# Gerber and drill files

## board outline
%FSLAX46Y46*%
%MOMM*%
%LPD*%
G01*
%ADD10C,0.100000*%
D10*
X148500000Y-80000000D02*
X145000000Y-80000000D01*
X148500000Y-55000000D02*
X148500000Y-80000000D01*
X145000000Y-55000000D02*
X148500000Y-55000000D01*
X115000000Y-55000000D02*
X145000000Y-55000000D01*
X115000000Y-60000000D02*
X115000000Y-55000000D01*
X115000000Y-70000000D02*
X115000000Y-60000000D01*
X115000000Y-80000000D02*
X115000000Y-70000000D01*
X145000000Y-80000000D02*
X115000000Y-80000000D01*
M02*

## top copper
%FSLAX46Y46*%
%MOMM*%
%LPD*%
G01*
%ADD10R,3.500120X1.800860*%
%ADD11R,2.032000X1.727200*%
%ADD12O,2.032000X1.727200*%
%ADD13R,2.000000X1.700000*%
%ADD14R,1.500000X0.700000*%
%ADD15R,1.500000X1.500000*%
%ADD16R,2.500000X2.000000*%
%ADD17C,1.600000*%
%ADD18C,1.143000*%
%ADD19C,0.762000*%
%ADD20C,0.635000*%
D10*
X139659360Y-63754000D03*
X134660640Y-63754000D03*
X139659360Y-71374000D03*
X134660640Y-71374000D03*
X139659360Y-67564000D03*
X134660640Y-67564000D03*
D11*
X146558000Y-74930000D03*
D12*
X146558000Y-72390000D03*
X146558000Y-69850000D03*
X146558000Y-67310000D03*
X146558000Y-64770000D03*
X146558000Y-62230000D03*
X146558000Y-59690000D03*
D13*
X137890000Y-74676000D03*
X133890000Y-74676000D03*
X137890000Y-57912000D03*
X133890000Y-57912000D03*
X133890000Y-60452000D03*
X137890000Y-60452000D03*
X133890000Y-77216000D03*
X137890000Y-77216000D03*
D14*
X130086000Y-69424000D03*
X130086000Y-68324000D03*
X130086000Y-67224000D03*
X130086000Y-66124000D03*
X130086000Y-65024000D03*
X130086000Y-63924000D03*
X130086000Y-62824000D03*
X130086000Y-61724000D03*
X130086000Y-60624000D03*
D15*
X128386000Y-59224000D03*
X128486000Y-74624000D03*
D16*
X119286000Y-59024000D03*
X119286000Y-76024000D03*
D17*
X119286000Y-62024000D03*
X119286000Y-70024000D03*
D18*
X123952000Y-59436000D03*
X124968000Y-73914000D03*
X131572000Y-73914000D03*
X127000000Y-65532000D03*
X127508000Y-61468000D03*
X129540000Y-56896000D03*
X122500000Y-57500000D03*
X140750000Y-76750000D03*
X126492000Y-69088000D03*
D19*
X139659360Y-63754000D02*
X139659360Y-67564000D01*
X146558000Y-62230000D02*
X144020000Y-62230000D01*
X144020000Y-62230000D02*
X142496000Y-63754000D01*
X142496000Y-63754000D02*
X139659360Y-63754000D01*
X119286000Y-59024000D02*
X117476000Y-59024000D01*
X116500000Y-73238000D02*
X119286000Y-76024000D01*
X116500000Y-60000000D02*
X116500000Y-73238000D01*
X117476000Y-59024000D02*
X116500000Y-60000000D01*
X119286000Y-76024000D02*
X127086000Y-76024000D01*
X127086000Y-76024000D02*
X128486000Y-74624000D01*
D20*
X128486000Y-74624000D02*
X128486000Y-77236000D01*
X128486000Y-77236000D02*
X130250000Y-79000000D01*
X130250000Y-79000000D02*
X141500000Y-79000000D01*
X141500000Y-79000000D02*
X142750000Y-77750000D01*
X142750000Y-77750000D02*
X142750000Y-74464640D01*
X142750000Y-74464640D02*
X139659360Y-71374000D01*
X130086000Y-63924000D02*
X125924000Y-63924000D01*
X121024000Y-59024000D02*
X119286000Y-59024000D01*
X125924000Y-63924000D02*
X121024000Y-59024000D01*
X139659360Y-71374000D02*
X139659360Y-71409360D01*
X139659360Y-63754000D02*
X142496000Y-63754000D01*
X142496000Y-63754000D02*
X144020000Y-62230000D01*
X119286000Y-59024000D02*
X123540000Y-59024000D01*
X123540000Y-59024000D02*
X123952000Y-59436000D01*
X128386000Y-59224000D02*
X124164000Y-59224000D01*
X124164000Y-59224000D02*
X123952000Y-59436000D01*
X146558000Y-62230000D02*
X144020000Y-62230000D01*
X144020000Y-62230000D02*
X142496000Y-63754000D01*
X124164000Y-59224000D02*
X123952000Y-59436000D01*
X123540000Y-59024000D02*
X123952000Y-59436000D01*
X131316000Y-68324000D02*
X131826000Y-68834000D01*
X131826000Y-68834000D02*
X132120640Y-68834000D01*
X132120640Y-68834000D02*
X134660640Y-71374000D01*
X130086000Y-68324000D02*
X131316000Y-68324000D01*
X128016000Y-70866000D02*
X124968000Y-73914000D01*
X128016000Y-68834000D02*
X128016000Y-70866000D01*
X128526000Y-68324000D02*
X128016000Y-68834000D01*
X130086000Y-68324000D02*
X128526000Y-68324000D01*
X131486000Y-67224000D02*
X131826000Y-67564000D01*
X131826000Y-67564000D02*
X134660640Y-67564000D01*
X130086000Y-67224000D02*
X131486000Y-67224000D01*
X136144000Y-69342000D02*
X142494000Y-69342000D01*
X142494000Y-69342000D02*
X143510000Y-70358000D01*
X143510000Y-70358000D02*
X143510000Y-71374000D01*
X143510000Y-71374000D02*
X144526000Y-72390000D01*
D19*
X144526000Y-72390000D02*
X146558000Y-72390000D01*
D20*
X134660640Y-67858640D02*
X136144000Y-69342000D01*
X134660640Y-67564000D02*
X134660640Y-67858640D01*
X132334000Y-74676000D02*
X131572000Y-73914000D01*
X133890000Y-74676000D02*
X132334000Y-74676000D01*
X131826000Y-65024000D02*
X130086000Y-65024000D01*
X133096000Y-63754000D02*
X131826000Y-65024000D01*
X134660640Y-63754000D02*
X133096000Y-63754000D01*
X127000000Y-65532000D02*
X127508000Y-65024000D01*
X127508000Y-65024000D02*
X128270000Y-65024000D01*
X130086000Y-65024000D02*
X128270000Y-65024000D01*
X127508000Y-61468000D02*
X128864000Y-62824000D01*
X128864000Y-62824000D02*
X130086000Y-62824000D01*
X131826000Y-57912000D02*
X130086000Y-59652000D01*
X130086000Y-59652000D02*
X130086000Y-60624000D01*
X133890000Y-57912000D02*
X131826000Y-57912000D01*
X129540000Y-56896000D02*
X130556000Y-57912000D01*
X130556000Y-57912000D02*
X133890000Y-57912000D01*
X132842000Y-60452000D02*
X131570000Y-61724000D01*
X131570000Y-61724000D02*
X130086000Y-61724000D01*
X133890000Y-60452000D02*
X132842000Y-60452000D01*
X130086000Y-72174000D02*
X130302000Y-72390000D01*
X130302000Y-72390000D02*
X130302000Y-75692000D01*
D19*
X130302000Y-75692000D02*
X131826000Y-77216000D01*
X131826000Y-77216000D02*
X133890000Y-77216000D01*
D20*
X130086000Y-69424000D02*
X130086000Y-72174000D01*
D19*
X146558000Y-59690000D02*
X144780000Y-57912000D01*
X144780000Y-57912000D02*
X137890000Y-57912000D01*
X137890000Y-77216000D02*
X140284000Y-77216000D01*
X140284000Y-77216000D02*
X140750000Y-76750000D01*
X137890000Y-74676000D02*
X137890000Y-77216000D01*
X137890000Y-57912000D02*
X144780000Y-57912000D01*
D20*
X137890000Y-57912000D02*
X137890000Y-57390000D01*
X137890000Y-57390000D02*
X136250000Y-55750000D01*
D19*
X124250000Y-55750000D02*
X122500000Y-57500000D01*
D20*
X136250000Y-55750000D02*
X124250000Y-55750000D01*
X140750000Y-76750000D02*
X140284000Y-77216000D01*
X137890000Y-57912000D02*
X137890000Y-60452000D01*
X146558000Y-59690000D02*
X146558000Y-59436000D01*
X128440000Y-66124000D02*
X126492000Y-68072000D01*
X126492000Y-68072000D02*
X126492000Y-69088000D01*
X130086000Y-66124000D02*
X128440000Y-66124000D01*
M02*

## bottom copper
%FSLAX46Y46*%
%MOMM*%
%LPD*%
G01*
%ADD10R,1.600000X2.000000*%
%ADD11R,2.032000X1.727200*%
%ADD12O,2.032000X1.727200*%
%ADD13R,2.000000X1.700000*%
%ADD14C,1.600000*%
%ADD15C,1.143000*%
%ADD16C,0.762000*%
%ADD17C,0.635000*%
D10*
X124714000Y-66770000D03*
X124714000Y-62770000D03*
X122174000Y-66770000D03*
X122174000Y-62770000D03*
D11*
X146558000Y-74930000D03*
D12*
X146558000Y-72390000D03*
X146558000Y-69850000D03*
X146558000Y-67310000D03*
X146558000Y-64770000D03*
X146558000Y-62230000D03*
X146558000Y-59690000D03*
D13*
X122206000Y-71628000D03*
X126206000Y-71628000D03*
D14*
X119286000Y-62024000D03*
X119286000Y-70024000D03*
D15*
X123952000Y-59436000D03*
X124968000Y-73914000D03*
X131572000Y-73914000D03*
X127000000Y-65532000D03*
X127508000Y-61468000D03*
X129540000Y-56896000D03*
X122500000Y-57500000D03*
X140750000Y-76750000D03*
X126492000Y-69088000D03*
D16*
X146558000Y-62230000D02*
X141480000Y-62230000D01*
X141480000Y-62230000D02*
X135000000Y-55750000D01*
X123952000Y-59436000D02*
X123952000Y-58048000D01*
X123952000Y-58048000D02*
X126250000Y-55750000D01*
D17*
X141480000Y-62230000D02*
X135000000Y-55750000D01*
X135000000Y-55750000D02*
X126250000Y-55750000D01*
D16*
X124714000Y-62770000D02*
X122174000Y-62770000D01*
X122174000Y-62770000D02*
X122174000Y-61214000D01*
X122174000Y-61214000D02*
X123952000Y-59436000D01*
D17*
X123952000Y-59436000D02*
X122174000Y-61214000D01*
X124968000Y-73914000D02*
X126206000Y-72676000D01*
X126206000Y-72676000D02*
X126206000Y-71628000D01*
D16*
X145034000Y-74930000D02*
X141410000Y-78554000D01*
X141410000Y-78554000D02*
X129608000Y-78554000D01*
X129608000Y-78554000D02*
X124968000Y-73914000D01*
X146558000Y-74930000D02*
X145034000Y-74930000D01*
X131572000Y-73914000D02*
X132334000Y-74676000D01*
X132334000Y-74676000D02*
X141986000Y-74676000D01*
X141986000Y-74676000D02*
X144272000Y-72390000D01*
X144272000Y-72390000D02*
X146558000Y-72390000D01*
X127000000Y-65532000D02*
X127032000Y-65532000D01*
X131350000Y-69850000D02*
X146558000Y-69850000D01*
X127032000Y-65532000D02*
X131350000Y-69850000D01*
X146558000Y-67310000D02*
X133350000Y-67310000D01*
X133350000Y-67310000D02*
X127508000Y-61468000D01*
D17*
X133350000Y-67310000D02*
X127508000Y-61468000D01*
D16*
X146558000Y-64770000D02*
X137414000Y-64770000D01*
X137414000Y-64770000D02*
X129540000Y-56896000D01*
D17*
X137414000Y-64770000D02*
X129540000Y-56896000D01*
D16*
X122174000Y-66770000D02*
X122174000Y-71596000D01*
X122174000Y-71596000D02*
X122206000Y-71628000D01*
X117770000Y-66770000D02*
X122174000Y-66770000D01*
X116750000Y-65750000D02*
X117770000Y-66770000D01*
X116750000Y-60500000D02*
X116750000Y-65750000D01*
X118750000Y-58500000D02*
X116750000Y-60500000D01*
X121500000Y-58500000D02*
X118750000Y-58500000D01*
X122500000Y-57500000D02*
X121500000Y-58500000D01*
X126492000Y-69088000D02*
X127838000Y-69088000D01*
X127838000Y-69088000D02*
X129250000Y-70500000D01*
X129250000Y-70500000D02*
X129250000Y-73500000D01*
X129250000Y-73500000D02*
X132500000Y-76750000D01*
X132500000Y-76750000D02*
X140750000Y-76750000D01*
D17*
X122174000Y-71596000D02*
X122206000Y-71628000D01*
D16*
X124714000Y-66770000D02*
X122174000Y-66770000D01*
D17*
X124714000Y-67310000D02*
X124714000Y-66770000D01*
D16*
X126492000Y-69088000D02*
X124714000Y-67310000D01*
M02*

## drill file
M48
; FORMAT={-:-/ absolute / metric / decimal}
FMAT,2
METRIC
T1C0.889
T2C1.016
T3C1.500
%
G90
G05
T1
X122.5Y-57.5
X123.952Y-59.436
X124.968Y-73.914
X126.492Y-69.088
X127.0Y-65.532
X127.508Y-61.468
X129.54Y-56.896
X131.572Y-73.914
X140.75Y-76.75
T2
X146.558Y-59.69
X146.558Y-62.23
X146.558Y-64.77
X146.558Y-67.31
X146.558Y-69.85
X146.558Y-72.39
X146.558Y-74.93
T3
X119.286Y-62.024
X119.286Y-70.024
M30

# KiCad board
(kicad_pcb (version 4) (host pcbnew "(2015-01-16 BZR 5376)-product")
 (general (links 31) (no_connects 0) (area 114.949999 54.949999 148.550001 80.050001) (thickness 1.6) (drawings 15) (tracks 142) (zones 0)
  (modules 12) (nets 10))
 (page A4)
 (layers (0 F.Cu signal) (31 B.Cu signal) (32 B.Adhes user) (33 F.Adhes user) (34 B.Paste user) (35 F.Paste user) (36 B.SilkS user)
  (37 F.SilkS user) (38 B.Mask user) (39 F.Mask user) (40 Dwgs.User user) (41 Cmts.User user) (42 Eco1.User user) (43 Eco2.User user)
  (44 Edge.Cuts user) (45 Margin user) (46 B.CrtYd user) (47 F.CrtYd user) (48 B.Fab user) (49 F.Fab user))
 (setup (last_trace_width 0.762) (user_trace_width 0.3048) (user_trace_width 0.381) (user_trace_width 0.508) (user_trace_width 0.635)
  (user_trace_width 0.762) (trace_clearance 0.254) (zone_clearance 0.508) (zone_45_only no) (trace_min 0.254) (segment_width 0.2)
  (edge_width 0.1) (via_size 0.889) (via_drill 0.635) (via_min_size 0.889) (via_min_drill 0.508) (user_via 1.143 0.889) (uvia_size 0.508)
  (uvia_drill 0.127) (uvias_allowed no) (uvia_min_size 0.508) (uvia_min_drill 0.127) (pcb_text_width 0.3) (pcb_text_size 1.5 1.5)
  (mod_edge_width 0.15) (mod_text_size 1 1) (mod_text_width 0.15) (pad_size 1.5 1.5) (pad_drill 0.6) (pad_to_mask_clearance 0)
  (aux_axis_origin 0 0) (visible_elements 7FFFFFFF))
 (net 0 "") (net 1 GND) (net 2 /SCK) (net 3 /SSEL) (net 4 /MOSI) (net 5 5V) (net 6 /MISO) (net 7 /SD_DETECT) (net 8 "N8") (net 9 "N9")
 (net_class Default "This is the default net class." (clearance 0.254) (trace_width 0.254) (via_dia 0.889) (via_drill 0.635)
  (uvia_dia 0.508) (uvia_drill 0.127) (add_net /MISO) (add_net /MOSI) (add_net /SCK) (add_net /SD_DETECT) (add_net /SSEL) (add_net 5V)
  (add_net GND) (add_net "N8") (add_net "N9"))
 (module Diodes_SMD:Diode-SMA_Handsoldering (layer F.Cu) (at 137.16 63.754 180)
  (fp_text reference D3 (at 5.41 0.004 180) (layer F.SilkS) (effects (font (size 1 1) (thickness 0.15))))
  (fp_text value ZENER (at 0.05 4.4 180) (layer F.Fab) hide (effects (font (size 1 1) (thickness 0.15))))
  (pad 1 smd rect (at -2.49936 0 180) (size 3.50012 1.80086) (layers F.Cu F.Paste F.Mask) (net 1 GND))
  (pad 2 smd rect (at 2.49936 0 180) (size 3.50012 1.80086) (layers F.Cu F.Paste F.Mask) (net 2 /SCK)))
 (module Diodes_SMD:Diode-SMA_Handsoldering (layer F.Cu) (at 137.16 71.374 180)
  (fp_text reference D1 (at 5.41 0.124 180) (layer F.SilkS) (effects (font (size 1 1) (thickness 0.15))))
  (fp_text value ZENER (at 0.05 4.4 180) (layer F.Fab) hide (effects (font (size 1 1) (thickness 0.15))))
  (pad 1 smd rect (at -2.49936 0 180) (size 3.50012 1.80086) (layers F.Cu F.Paste F.Mask) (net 1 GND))
  (pad 2 smd rect (at 2.49936 0 180) (size 3.50012 1.80086) (layers F.Cu F.Paste F.Mask) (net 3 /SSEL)))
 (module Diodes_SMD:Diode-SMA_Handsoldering (layer F.Cu) (at 137.16 67.564 180)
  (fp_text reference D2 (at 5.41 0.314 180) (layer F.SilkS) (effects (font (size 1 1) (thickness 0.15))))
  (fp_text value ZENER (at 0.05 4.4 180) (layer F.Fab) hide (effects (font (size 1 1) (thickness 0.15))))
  (pad 1 smd rect (at -2.49936 0 180) (size 3.50012 1.80086) (layers F.Cu F.Paste F.Mask) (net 1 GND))
  (pad 2 smd rect (at 2.49936 0 180) (size 3.50012 1.80086) (layers F.Cu F.Paste F.Mask) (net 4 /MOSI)))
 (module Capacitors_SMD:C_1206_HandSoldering (layer B.Cu) (at 124.714 64.77 90)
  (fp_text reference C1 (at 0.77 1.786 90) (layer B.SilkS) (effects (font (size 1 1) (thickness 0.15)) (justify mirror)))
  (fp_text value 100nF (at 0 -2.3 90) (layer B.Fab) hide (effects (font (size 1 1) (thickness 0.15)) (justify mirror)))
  (pad 1 smd rect (at -2 0 90) (size 2 1.6) (layers B.Cu B.Paste B.Mask) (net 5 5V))
  (pad 2 smd rect (at 2 0 90) (size 2 1.6) (layers B.Cu B.Paste B.Mask) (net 1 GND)))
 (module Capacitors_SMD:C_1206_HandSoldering (layer B.Cu) (at 122.174 64.77 90)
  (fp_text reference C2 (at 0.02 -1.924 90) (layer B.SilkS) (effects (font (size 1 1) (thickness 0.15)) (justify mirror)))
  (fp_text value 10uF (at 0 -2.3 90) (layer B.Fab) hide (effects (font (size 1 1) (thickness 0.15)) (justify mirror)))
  (pad 1 smd rect (at -2 0 90) (size 2 1.6) (layers B.Cu B.Paste B.Mask) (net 5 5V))
  (pad 2 smd rect (at 2 0 90) (size 2 1.6) (layers B.Cu B.Paste B.Mask) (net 1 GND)))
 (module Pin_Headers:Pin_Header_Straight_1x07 (layer F.Cu) (at 146.558 74.93 180)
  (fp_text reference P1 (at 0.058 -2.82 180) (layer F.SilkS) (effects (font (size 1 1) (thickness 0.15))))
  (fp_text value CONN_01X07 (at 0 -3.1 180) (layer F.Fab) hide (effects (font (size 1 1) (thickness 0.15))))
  (pad 1 thru_hole rect (at 0 0 180) (size 2.032 1.7272) (drill 1.016) (layers *.Cu *.Mask F.SilkS) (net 3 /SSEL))
  (pad 2 thru_hole oval (at 0 2.54 180) (size 2.032 1.7272) (drill 1.016) (layers *.Cu *.Mask F.SilkS) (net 4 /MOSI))
  (pad 3 thru_hole oval (at 0 5.08 180) (size 2.032 1.7272) (drill 1.016) (layers *.Cu *.Mask F.SilkS) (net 2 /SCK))
  (pad 4 thru_hole oval (at 0 7.62 180) (size 2.032 1.7272) (drill 1.016) (layers *.Cu *.Mask F.SilkS) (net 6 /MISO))
  (pad 5 thru_hole oval (at 0 10.16 180) (size 2.032 1.7272) (drill 1.016) (layers *.Cu *.Mask F.SilkS) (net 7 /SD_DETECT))
  (pad 6 thru_hole oval (at 0 12.7 180) (size 2.032 1.7272) (drill 1.016) (layers *.Cu *.Mask F.SilkS) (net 1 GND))
  (pad 7 thru_hole oval (at 0 15.24 180) (size 2.032 1.7272) (drill 1.016) (layers *.Cu *.Mask F.SilkS) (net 5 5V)))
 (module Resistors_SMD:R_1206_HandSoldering (layer B.Cu) (at 124.206 71.628)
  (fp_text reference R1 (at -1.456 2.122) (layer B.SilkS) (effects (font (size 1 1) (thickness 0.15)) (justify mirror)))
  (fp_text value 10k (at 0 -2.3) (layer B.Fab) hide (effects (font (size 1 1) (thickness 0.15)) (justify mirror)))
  (pad 1 smd rect (at -2 0) (size 2 1.7) (layers B.Cu B.Paste B.Mask) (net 5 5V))
  (pad 2 smd rect (at 2 0) (size 2 1.7) (layers B.Cu B.Paste B.Mask) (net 3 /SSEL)))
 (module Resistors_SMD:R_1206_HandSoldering (layer F.Cu) (at 135.89 74.676 180)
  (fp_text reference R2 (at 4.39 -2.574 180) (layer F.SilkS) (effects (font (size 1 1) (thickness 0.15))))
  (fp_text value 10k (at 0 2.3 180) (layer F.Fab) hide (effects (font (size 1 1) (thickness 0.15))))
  (pad 1 smd rect (at -2 0 180) (size 2 1.7) (layers F.Cu F.Paste F.Mask) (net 5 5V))
  (pad 2 smd rect (at 2 0 180) (size 2 1.7) (layers F.Cu F.Paste F.Mask) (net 4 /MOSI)))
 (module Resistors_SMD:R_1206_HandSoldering (layer F.Cu) (at 135.89 57.912 180)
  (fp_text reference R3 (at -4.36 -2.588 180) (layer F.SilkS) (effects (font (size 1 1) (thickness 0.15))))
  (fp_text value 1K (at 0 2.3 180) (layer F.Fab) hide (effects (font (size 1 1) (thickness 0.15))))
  (pad 1 smd rect (at -2 0 180) (size 2 1.7) (layers F.Cu F.Paste F.Mask) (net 5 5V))
  (pad 2 smd rect (at 2 0 180) (size 2 1.7) (layers F.Cu F.Paste F.Mask) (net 7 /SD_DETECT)))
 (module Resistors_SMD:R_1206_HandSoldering (layer F.Cu) (at 135.89 60.452)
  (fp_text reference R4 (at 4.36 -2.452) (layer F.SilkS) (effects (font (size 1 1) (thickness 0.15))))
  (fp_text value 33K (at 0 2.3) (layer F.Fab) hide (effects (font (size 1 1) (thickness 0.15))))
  (pad 1 smd rect (at -2 0) (size 2 1.7) (layers F.Cu F.Paste F.Mask) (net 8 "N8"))
  (pad 2 smd rect (at 2 0) (size 2 1.7) (layers F.Cu F.Paste F.Mask) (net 5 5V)))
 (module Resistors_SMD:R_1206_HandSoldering (layer F.Cu) (at 135.89 77.216)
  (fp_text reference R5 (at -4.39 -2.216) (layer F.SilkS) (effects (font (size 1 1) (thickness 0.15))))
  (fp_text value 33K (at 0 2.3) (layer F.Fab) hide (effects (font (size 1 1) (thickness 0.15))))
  (pad 1 smd rect (at -2 0) (size 2 1.7) (layers F.Cu F.Paste F.Mask) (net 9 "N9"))
  (pad 2 smd rect (at 2 0) (size 2 1.7) (layers F.Cu F.Paste F.Mask) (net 5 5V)))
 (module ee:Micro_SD (layer F.Cu) (at 129.286 65.024 270)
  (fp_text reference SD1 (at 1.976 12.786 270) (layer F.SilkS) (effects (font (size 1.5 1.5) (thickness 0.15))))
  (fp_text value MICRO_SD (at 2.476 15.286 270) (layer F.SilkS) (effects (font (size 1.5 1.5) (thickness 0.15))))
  (pad 1 smd rect (at 4.4 -0.8 270) (size 0.7 1.5) (layers F.Cu F.Paste F.Mask) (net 9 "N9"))
  (pad 2 smd rect (at 3.3 -0.8 270) (size 0.7 1.5) (layers F.Cu F.Paste F.Mask) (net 3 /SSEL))
  (pad 3 smd rect (at 2.2 -0.8 270) (size 0.7 1.5) (layers F.Cu F.Paste F.Mask) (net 4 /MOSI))
  (pad 4 smd rect (at 1.1 -0.8 270) (size 0.7 1.5) (layers F.Cu F.Paste F.Mask) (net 5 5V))
  (pad 5 smd rect (at 0 -0.8 270) (size 0.7 1.5) (layers F.Cu F.Paste F.Mask) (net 2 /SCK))
  (pad 6 smd rect (at -1.1 -0.8 270) (size 0.7 1.5) (layers F.Cu F.Paste F.Mask) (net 1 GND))
  (pad 7 smd rect (at -2.2 -0.8 270) (size 0.7 1.5) (layers F.Cu F.Paste F.Mask) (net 6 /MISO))
  (pad 8 smd rect (at -3.3 -0.8 270) (size 0.7 1.5) (layers F.Cu F.Paste F.Mask) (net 8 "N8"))
  (pad 9 smd rect (at -4.4 -0.8 270) (size 0.7 1.5) (layers F.Cu F.Paste F.Mask) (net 7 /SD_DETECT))
  (pad 10 smd rect (at -5.8 0.9 270) (size 1.5 1.5) (layers F.Cu F.Paste F.Mask) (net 1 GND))
  (pad 11 smd rect (at 9.6 0.8 270) (size 1.5 1.5) (layers F.Cu F.Paste F.Mask) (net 1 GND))
  (pad 12 smd rect (at -6 10 270) (size 2 2.5) (layers F.Cu F.Paste F.Mask) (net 1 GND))
  (pad 13 smd rect (at 11 10 270) (size 2 2.5) (layers F.Cu F.Paste F.Mask) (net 1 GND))
  (pad "" thru_hole circle (at -3 10 270) (size 1.6 1.6) (drill 1.5) (layers *.Cu *.Mask F.SilkS))
  (pad "" thru_hole circle (at 5 10 270) (size 1.6 1.6) (drill 1.5) (layers *.Cu *.Mask F.SilkS)))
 (gr_line (start 148.5 80) (end 145 80) (angle 90) (layer Edge.Cuts) (width 0.1))
 (gr_line (start 148.5 55) (end 148.5 80) (angle 90) (layer Edge.Cuts) (width 0.1))
 (gr_line (start 145 55) (end 148.5 55) (angle 90) (layer Edge.Cuts) (width 0.1))
 (gr_line (start 115 55) (end 145 55) (angle 90) (layer Edge.Cuts) (width 0.1))
 (gr_line (start 115 60) (end 115 55) (angle 90) (layer Edge.Cuts) (width 0.1))
 (gr_line (start 115 70) (end 115 60) (angle 90) (layer Edge.Cuts) (width 0.1))
 (gr_line (start 115 80) (end 115 70) (angle 90) (layer Edge.Cuts) (width 0.1))
 (gr_line (start 145 80) (end 115 80) (angle 90) (layer Edge.Cuts) (width 0.1))
 (segment (start 146.558 62.23) (end 141.48 62.23) (width 0.762) (layer B.Cu) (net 1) (status 400000))
 (segment (start 141.48 62.23) (end 135 55.75) (width 0.762) (layer B.Cu) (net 1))
 (segment (start 123.952 59.436) (end 123.952 58.048) (width 0.762) (layer B.Cu) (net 1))
 (segment (start 123.952 58.048) (end 126.25 55.75) (width 0.762) (layer B.Cu) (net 1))
 (segment (start 141.48 62.23) (end 135 55.75) (width 0.635) (layer B.Cu) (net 1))
 (segment (start 135 55.75) (end 126.25 55.75) (width 0.635) (layer B.Cu) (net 1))
 (segment (start 139.65936 63.754) (end 139.65936 67.564) (width 0.762) (layer F.Cu) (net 1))
 (segment (start 146.558 62.23) (end 144.02 62.23) (width 0.762) (layer F.Cu) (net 1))
 (segment (start 144.02 62.23) (end 142.496 63.754) (width 0.762) (layer F.Cu) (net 1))
 (segment (start 142.496 63.754) (end 139.65936 63.754) (width 0.762) (layer F.Cu) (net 1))
 (segment (start 119.286 59.024) (end 117.476 59.024) (width 0.762) (layer F.Cu) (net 1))
 (segment (start 116.5 73.238) (end 119.286 76.024) (width 0.762) (layer F.Cu) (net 1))
 (segment (start 116.5 60) (end 116.5 73.238) (width 0.762) (layer F.Cu) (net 1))
 (segment (start 117.476 59.024) (end 116.5 60) (width 0.762) (layer F.Cu) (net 1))
 (segment (start 119.286 76.024) (end 127.086 76.024) (width 0.762) (layer F.Cu) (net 1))
 (segment (start 127.086 76.024) (end 128.486 74.624) (width 0.762) (layer F.Cu) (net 1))
 (segment (start 128.486 74.624) (end 128.486 77.236) (width 0.635) (layer F.Cu) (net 1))
 (segment (start 128.486 77.236) (end 130.25 79) (width 0.635) (layer F.Cu) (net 1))
 (segment (start 130.25 79) (end 141.5 79) (width 0.635) (layer F.Cu) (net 1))
 (segment (start 141.5 79) (end 142.75 77.75) (width 0.635) (layer F.Cu) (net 1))
 (segment (start 142.75 77.75) (end 142.75 74.46464) (width 0.635) (layer F.Cu) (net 1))
 (segment (start 142.75 74.46464) (end 139.65936 71.374) (width 0.635) (layer F.Cu) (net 1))
 (segment (start 130.086 63.924) (end 125.924 63.924) (width 0.635) (layer F.Cu) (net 1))
 (segment (start 121.024 59.024) (end 119.286 59.024) (width 0.635) (layer F.Cu) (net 1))
 (segment (start 125.924 63.924) (end 121.024 59.024) (width 0.635) (layer F.Cu) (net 1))
 (segment (start 139.65936 71.374) (end 139.65936 71.40936) (width 0.635) (layer F.Cu) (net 1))
 (segment (start 139.65936 63.754) (end 142.496 63.754) (width 0.635) (layer F.Cu) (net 1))
 (segment (start 142.496 63.754) (end 144.02 62.23) (width 0.635) (layer F.Cu) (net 1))
 (segment (start 124.714 62.77) (end 122.174 62.77) (width 0.762) (layer B.Cu) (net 1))
 (segment (start 122.174 62.77) (end 122.174 61.214) (width 0.762) (layer B.Cu) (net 1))
 (segment (start 122.174 61.214) (end 123.952 59.436) (width 0.762) (layer B.Cu) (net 1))
 (segment (start 119.286 59.024) (end 123.54 59.024) (width 0.635) (layer F.Cu) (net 1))
 (segment (start 123.54 59.024) (end 123.952 59.436) (width 0.635) (layer F.Cu) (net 1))
 (segment (start 128.386 59.224) (end 124.164 59.224) (width 0.635) (layer F.Cu) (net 1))
 (segment (start 124.164 59.224) (end 123.952 59.436) (width 0.635) (layer F.Cu) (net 1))
 (segment (start 146.558 62.23) (end 144.02 62.23) (width 0.635) (layer F.Cu) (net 1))
 (segment (start 144.02 62.23) (end 142.496 63.754) (width 0.635) (layer F.Cu) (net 1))
 (segment (start 123.952 59.436) (end 122.174 61.214) (width 0.635) (layer B.Cu) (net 1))
 (via (at 123.952 59.436) (size 1.143) (drill 0.889) (layers F.Cu B.Cu) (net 1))
 (segment (start 124.164 59.224) (end 123.952 59.436) (width 0.635) (layer F.Cu) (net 1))
 (segment (start 123.54 59.024) (end 123.952 59.436) (width 0.635) (layer F.Cu) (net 1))
 (segment (start 131.316 68.324) (end 131.826 68.834) (width 0.635) (layer F.Cu) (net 3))
 (segment (start 131.826 68.834) (end 132.12064 68.834) (width 0.635) (layer F.Cu) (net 3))
 (segment (start 132.12064 68.834) (end 134.66064 71.374) (width 0.635) (layer F.Cu) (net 3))
 (segment (start 130.086 68.324) (end 131.316 68.324) (width 0.635) (layer F.Cu) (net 3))
 (segment (start 124.968 73.914) (end 126.206 72.676) (width 0.635) (layer B.Cu) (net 3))
 (segment (start 126.206 72.676) (end 126.206 71.628) (width 0.635) (layer B.Cu) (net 3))
 (via (at 124.968 73.914) (size 1.143) (drill 0.889) (layers F.Cu B.Cu) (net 3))
 (segment (start 128.016 70.866) (end 124.968 73.914) (width 0.635) (layer F.Cu) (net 3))
 (segment (start 128.016 68.834) (end 128.016 70.866) (width 0.635) (layer F.Cu) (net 3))
 (segment (start 128.526 68.324) (end 128.016 68.834) (width 0.635) (layer F.Cu) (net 3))
 (segment (start 130.086 68.324) (end 128.526 68.324) (width 0.635) (layer F.Cu) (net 3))
 (segment (start 145.034 74.93) (end 141.41 78.554) (width 0.762) (layer B.Cu) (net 3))
 (segment (start 141.41 78.554) (end 129.608 78.554) (width 0.762) (layer B.Cu) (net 3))
 (segment (start 129.608 78.554) (end 124.968 73.914) (width 0.762) (layer B.Cu) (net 3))
 (segment (start 146.558 74.93) (end 145.034 74.93) (width 0.762) (layer B.Cu) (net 3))
 (segment (start 131.486 67.224) (end 131.826 67.564) (width 0.635) (layer F.Cu) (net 4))
 (segment (start 131.826 67.564) (end 134.66064 67.564) (width 0.635) (layer F.Cu) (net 4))
 (segment (start 130.086 67.224) (end 131.486 67.224) (width 0.635) (layer F.Cu) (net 4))
 (segment (start 136.144 69.342) (end 142.494 69.342) (width 0.635) (layer F.Cu) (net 4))
 (segment (start 142.494 69.342) (end 143.51 70.358) (width 0.635) (layer F.Cu) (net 4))
 (segment (start 143.51 70.358) (end 143.51 71.374) (width 0.635) (layer F.Cu) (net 4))
 (segment (start 143.51 71.374) (end 144.526 72.39) (width 0.635) (layer F.Cu) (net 4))
 (segment (start 144.526 72.39) (end 146.558 72.39) (width 0.762) (layer F.Cu) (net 4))
 (segment (start 134.66064 67.85864) (end 136.144 69.342) (width 0.635) (layer F.Cu) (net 4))
 (segment (start 134.66064 67.564) (end 134.66064 67.85864) (width 0.635) (layer F.Cu) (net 4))
 (segment (start 132.334 74.676) (end 131.572 73.914) (width 0.635) (layer F.Cu) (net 4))
 (via (at 131.572 73.914) (size 1.143) (drill 0.889) (layers F.Cu B.Cu) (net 4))
 (segment (start 131.572 73.914) (end 132.334 74.676) (width 0.762) (layer B.Cu) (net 4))
 (segment (start 132.334 74.676) (end 141.986 74.676) (width 0.762) (layer B.Cu) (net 4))
 (segment (start 141.986 74.676) (end 144.272 72.39) (width 0.762) (layer B.Cu) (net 4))
 (segment (start 144.272 72.39) (end 146.558 72.39) (width 0.762) (layer B.Cu) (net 4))
 (segment (start 133.89 74.676) (end 132.334 74.676) (width 0.635) (layer F.Cu) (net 4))
 (segment (start 127 65.532) (end 127.032 65.532) (width 0.762) (layer B.Cu) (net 2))
 (segment (start 131.35 69.85) (end 146.558 69.85) (width 0.762) (layer B.Cu) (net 2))
 (segment (start 127.032 65.532) (end 131.35 69.85) (width 0.762) (layer B.Cu) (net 2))
 (segment (start 131.826 65.024) (end 130.086 65.024) (width 0.635) (layer F.Cu) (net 2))
 (segment (start 133.096 63.754) (end 131.826 65.024) (width 0.635) (layer F.Cu) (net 2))
 (segment (start 134.66064 63.754) (end 133.096 63.754) (width 0.635) (layer F.Cu) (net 2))
 (via (at 127 65.532) (size 1.143) (drill 0.889) (layers F.Cu B.Cu) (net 2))
 (segment (start 127 65.532) (end 127.508 65.024) (width 0.635) (layer F.Cu) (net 2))
 (segment (start 127.508 65.024) (end 128.27 65.024) (width 0.635) (layer F.Cu) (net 2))
 (segment (start 130.086 65.024) (end 128.27 65.024) (width 0.635) (layer F.Cu) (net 2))
 (segment (start 146.558 67.31) (end 133.35 67.31) (width 0.762) (layer B.Cu) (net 6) (status 400000))
 (segment (start 133.35 67.31) (end 127.508 61.468) (width 0.762) (layer B.Cu) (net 6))
 (segment (start 133.35 67.31) (end 127.508 61.468) (width 0.635) (layer B.Cu) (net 6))
 (via (at 127.508 61.468) (size 1.143) (drill 0.889) (layers F.Cu B.Cu) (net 6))
 (segment (start 127.508 61.468) (end 128.864 62.824) (width 0.635) (layer F.Cu) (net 6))
 (segment (start 128.864 62.824) (end 130.086 62.824) (width 0.635) (layer F.Cu) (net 6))
 (segment (start 146.558 64.77) (end 137.414 64.77) (width 0.762) (layer B.Cu) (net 7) (status 400000))
 (segment (start 137.414 64.77) (end 129.54 56.896) (width 0.762) (layer B.Cu) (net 7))
 (segment (start 131.826 57.912) (end 130.086 59.652) (width 0.635) (layer F.Cu) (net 7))
 (segment (start 130.086 59.652) (end 130.086 60.624) (width 0.635) (layer F.Cu) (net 7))
 (segment (start 133.89 57.912) (end 131.826 57.912) (width 0.635) (layer F.Cu) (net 7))
 (segment (start 137.414 64.77) (end 129.54 56.896) (width 0.635) (layer B.Cu) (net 7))
 (via (at 129.54 56.896) (size 1.143) (drill 0.889) (layers F.Cu B.Cu) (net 7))
 (segment (start 129.54 56.896) (end 130.556 57.912) (width 0.635) (layer F.Cu) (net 7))
 (segment (start 130.556 57.912) (end 133.89 57.912) (width 0.635) (layer F.Cu) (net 7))
 (segment (start 132.842 60.452) (end 131.57 61.724) (width 0.635) (layer F.Cu) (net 8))
 (segment (start 131.57 61.724) (end 130.086 61.724) (width 0.635) (layer F.Cu) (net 8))
 (segment (start 133.89 60.452) (end 132.842 60.452) (width 0.635) (layer F.Cu) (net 8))
 (segment (start 130.086 72.174) (end 130.302 72.39) (width 0.635) (layer F.Cu) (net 9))
 (segment (start 130.302 72.39) (end 130.302 75.692) (width 0.635) (layer F.Cu) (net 9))
 (segment (start 130.302 75.692) (end 131.826 77.216) (width 0.762) (layer F.Cu) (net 9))
 (segment (start 131.826 77.216) (end 133.89 77.216) (width 0.762) (layer F.Cu) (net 9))
 (segment (start 130.086 69.424) (end 130.086 72.174) (width 0.635) (layer F.Cu) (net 9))
 (segment (start 122.174 66.77) (end 122.174 71.596) (width 0.762) (layer B.Cu) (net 5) (status C00000))
 (segment (start 122.174 71.596) (end 122.206 71.628) (width 0.762) (layer B.Cu) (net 5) (status C00000))
 (segment (start 146.558 59.69) (end 144.78 57.912) (width 0.762) (layer F.Cu) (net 5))
 (segment (start 144.78 57.912) (end 137.89 57.912) (width 0.762) (layer F.Cu) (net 5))
 (segment (start 137.89 77.216) (end 140.284 77.216) (width 0.762) (layer F.Cu) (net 5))
 (segment (start 140.284 77.216) (end 140.75 76.75) (width 0.762) (layer F.Cu) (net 5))
 (segment (start 137.89 74.676) (end 137.89 77.216) (width 0.762) (layer F.Cu) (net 5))
 (segment (start 137.89 57.912) (end 144.78 57.912) (width 0.762) (layer F.Cu) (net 5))
 (segment (start 137.89 57.912) (end 137.89 57.39) (width 0.635) (layer F.Cu) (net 5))
 (segment (start 137.89 57.39) (end 136.25 55.75) (width 0.635) (layer F.Cu) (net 5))
 (segment (start 117.77 66.77) (end 122.174 66.77) (width 0.762) (layer B.Cu) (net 5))
 (segment (start 116.75 65.75) (end 117.77 66.77) (width 0.762) (layer B.Cu) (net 5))
 (segment (start 116.75 60.5) (end 116.75 65.75) (width 0.762) (layer B.Cu) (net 5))
 (segment (start 118.75 58.5) (end 116.75 60.5) (width 0.762) (layer B.Cu) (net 5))
 (segment (start 121.5 58.5) (end 118.75 58.5) (width 0.762) (layer B.Cu) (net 5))
 (segment (start 122.5 57.5) (end 121.5 58.5) (width 0.762) (layer B.Cu) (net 5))
 (via (at 122.5 57.5) (size 1.143) (drill 0.889) (layers F.Cu B.Cu) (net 5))
 (segment (start 124.25 55.75) (end 122.5 57.5) (width 0.762) (layer F.Cu) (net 5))
 (segment (start 136.25 55.75) (end 124.25 55.75) (width 0.635) (layer F.Cu) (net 5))
 (segment (start 126.492 69.088) (end 127.838 69.088) (width 0.762) (layer B.Cu) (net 5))
 (segment (start 127.838 69.088) (end 129.25 70.5) (width 0.762) (layer B.Cu) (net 5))
 (segment (start 129.25 70.5) (end 129.25 73.5) (width 0.762) (layer B.Cu) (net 5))
 (segment (start 129.25 73.5) (end 132.5 76.75) (width 0.762) (layer B.Cu) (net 5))
 (segment (start 132.5 76.75) (end 140.75 76.75) (width 0.762) (layer B.Cu) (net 5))
 (via (at 140.75 76.75) (size 1.143) (drill 0.889) (layers F.Cu B.Cu) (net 5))
 (segment (start 140.75 76.75) (end 140.284 77.216) (width 0.635) (layer F.Cu) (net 5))
 (segment (start 122.174 71.596) (end 122.206 71.628) (width 0.635) (layer B.Cu) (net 5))
 (segment (start 137.89 57.912) (end 137.89 60.452) (width 0.635) (layer F.Cu) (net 5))
 (segment (start 124.714 66.77) (end 122.174 66.77) (width 0.762) (layer B.Cu) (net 5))
 (segment (start 146.558 59.69) (end 146.558 59.436) (width 0.635) (layer F.Cu) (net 5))
 (segment (start 124.714 67.31) (end 124.714 66.77) (width 0.635) (layer B.Cu) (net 5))
 (segment (start 128.44 66.124) (end 126.492 68.072) (width 0.635) (layer F.Cu) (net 5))
 (segment (start 126.492 68.072) (end 126.492 69.088) (width 0.635) (layer F.Cu) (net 5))
 (via (at 126.492 69.088) (size 1.143) (drill 0.889) (layers F.Cu B.Cu) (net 5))
 (segment (start 126.492 69.088) (end 124.714 67.31) (width 0.762) (layer B.Cu) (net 5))
 (segment (start 130.086 66.124) (end 128.44 66.124) (width 0.635) (layer F.Cu) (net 5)))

